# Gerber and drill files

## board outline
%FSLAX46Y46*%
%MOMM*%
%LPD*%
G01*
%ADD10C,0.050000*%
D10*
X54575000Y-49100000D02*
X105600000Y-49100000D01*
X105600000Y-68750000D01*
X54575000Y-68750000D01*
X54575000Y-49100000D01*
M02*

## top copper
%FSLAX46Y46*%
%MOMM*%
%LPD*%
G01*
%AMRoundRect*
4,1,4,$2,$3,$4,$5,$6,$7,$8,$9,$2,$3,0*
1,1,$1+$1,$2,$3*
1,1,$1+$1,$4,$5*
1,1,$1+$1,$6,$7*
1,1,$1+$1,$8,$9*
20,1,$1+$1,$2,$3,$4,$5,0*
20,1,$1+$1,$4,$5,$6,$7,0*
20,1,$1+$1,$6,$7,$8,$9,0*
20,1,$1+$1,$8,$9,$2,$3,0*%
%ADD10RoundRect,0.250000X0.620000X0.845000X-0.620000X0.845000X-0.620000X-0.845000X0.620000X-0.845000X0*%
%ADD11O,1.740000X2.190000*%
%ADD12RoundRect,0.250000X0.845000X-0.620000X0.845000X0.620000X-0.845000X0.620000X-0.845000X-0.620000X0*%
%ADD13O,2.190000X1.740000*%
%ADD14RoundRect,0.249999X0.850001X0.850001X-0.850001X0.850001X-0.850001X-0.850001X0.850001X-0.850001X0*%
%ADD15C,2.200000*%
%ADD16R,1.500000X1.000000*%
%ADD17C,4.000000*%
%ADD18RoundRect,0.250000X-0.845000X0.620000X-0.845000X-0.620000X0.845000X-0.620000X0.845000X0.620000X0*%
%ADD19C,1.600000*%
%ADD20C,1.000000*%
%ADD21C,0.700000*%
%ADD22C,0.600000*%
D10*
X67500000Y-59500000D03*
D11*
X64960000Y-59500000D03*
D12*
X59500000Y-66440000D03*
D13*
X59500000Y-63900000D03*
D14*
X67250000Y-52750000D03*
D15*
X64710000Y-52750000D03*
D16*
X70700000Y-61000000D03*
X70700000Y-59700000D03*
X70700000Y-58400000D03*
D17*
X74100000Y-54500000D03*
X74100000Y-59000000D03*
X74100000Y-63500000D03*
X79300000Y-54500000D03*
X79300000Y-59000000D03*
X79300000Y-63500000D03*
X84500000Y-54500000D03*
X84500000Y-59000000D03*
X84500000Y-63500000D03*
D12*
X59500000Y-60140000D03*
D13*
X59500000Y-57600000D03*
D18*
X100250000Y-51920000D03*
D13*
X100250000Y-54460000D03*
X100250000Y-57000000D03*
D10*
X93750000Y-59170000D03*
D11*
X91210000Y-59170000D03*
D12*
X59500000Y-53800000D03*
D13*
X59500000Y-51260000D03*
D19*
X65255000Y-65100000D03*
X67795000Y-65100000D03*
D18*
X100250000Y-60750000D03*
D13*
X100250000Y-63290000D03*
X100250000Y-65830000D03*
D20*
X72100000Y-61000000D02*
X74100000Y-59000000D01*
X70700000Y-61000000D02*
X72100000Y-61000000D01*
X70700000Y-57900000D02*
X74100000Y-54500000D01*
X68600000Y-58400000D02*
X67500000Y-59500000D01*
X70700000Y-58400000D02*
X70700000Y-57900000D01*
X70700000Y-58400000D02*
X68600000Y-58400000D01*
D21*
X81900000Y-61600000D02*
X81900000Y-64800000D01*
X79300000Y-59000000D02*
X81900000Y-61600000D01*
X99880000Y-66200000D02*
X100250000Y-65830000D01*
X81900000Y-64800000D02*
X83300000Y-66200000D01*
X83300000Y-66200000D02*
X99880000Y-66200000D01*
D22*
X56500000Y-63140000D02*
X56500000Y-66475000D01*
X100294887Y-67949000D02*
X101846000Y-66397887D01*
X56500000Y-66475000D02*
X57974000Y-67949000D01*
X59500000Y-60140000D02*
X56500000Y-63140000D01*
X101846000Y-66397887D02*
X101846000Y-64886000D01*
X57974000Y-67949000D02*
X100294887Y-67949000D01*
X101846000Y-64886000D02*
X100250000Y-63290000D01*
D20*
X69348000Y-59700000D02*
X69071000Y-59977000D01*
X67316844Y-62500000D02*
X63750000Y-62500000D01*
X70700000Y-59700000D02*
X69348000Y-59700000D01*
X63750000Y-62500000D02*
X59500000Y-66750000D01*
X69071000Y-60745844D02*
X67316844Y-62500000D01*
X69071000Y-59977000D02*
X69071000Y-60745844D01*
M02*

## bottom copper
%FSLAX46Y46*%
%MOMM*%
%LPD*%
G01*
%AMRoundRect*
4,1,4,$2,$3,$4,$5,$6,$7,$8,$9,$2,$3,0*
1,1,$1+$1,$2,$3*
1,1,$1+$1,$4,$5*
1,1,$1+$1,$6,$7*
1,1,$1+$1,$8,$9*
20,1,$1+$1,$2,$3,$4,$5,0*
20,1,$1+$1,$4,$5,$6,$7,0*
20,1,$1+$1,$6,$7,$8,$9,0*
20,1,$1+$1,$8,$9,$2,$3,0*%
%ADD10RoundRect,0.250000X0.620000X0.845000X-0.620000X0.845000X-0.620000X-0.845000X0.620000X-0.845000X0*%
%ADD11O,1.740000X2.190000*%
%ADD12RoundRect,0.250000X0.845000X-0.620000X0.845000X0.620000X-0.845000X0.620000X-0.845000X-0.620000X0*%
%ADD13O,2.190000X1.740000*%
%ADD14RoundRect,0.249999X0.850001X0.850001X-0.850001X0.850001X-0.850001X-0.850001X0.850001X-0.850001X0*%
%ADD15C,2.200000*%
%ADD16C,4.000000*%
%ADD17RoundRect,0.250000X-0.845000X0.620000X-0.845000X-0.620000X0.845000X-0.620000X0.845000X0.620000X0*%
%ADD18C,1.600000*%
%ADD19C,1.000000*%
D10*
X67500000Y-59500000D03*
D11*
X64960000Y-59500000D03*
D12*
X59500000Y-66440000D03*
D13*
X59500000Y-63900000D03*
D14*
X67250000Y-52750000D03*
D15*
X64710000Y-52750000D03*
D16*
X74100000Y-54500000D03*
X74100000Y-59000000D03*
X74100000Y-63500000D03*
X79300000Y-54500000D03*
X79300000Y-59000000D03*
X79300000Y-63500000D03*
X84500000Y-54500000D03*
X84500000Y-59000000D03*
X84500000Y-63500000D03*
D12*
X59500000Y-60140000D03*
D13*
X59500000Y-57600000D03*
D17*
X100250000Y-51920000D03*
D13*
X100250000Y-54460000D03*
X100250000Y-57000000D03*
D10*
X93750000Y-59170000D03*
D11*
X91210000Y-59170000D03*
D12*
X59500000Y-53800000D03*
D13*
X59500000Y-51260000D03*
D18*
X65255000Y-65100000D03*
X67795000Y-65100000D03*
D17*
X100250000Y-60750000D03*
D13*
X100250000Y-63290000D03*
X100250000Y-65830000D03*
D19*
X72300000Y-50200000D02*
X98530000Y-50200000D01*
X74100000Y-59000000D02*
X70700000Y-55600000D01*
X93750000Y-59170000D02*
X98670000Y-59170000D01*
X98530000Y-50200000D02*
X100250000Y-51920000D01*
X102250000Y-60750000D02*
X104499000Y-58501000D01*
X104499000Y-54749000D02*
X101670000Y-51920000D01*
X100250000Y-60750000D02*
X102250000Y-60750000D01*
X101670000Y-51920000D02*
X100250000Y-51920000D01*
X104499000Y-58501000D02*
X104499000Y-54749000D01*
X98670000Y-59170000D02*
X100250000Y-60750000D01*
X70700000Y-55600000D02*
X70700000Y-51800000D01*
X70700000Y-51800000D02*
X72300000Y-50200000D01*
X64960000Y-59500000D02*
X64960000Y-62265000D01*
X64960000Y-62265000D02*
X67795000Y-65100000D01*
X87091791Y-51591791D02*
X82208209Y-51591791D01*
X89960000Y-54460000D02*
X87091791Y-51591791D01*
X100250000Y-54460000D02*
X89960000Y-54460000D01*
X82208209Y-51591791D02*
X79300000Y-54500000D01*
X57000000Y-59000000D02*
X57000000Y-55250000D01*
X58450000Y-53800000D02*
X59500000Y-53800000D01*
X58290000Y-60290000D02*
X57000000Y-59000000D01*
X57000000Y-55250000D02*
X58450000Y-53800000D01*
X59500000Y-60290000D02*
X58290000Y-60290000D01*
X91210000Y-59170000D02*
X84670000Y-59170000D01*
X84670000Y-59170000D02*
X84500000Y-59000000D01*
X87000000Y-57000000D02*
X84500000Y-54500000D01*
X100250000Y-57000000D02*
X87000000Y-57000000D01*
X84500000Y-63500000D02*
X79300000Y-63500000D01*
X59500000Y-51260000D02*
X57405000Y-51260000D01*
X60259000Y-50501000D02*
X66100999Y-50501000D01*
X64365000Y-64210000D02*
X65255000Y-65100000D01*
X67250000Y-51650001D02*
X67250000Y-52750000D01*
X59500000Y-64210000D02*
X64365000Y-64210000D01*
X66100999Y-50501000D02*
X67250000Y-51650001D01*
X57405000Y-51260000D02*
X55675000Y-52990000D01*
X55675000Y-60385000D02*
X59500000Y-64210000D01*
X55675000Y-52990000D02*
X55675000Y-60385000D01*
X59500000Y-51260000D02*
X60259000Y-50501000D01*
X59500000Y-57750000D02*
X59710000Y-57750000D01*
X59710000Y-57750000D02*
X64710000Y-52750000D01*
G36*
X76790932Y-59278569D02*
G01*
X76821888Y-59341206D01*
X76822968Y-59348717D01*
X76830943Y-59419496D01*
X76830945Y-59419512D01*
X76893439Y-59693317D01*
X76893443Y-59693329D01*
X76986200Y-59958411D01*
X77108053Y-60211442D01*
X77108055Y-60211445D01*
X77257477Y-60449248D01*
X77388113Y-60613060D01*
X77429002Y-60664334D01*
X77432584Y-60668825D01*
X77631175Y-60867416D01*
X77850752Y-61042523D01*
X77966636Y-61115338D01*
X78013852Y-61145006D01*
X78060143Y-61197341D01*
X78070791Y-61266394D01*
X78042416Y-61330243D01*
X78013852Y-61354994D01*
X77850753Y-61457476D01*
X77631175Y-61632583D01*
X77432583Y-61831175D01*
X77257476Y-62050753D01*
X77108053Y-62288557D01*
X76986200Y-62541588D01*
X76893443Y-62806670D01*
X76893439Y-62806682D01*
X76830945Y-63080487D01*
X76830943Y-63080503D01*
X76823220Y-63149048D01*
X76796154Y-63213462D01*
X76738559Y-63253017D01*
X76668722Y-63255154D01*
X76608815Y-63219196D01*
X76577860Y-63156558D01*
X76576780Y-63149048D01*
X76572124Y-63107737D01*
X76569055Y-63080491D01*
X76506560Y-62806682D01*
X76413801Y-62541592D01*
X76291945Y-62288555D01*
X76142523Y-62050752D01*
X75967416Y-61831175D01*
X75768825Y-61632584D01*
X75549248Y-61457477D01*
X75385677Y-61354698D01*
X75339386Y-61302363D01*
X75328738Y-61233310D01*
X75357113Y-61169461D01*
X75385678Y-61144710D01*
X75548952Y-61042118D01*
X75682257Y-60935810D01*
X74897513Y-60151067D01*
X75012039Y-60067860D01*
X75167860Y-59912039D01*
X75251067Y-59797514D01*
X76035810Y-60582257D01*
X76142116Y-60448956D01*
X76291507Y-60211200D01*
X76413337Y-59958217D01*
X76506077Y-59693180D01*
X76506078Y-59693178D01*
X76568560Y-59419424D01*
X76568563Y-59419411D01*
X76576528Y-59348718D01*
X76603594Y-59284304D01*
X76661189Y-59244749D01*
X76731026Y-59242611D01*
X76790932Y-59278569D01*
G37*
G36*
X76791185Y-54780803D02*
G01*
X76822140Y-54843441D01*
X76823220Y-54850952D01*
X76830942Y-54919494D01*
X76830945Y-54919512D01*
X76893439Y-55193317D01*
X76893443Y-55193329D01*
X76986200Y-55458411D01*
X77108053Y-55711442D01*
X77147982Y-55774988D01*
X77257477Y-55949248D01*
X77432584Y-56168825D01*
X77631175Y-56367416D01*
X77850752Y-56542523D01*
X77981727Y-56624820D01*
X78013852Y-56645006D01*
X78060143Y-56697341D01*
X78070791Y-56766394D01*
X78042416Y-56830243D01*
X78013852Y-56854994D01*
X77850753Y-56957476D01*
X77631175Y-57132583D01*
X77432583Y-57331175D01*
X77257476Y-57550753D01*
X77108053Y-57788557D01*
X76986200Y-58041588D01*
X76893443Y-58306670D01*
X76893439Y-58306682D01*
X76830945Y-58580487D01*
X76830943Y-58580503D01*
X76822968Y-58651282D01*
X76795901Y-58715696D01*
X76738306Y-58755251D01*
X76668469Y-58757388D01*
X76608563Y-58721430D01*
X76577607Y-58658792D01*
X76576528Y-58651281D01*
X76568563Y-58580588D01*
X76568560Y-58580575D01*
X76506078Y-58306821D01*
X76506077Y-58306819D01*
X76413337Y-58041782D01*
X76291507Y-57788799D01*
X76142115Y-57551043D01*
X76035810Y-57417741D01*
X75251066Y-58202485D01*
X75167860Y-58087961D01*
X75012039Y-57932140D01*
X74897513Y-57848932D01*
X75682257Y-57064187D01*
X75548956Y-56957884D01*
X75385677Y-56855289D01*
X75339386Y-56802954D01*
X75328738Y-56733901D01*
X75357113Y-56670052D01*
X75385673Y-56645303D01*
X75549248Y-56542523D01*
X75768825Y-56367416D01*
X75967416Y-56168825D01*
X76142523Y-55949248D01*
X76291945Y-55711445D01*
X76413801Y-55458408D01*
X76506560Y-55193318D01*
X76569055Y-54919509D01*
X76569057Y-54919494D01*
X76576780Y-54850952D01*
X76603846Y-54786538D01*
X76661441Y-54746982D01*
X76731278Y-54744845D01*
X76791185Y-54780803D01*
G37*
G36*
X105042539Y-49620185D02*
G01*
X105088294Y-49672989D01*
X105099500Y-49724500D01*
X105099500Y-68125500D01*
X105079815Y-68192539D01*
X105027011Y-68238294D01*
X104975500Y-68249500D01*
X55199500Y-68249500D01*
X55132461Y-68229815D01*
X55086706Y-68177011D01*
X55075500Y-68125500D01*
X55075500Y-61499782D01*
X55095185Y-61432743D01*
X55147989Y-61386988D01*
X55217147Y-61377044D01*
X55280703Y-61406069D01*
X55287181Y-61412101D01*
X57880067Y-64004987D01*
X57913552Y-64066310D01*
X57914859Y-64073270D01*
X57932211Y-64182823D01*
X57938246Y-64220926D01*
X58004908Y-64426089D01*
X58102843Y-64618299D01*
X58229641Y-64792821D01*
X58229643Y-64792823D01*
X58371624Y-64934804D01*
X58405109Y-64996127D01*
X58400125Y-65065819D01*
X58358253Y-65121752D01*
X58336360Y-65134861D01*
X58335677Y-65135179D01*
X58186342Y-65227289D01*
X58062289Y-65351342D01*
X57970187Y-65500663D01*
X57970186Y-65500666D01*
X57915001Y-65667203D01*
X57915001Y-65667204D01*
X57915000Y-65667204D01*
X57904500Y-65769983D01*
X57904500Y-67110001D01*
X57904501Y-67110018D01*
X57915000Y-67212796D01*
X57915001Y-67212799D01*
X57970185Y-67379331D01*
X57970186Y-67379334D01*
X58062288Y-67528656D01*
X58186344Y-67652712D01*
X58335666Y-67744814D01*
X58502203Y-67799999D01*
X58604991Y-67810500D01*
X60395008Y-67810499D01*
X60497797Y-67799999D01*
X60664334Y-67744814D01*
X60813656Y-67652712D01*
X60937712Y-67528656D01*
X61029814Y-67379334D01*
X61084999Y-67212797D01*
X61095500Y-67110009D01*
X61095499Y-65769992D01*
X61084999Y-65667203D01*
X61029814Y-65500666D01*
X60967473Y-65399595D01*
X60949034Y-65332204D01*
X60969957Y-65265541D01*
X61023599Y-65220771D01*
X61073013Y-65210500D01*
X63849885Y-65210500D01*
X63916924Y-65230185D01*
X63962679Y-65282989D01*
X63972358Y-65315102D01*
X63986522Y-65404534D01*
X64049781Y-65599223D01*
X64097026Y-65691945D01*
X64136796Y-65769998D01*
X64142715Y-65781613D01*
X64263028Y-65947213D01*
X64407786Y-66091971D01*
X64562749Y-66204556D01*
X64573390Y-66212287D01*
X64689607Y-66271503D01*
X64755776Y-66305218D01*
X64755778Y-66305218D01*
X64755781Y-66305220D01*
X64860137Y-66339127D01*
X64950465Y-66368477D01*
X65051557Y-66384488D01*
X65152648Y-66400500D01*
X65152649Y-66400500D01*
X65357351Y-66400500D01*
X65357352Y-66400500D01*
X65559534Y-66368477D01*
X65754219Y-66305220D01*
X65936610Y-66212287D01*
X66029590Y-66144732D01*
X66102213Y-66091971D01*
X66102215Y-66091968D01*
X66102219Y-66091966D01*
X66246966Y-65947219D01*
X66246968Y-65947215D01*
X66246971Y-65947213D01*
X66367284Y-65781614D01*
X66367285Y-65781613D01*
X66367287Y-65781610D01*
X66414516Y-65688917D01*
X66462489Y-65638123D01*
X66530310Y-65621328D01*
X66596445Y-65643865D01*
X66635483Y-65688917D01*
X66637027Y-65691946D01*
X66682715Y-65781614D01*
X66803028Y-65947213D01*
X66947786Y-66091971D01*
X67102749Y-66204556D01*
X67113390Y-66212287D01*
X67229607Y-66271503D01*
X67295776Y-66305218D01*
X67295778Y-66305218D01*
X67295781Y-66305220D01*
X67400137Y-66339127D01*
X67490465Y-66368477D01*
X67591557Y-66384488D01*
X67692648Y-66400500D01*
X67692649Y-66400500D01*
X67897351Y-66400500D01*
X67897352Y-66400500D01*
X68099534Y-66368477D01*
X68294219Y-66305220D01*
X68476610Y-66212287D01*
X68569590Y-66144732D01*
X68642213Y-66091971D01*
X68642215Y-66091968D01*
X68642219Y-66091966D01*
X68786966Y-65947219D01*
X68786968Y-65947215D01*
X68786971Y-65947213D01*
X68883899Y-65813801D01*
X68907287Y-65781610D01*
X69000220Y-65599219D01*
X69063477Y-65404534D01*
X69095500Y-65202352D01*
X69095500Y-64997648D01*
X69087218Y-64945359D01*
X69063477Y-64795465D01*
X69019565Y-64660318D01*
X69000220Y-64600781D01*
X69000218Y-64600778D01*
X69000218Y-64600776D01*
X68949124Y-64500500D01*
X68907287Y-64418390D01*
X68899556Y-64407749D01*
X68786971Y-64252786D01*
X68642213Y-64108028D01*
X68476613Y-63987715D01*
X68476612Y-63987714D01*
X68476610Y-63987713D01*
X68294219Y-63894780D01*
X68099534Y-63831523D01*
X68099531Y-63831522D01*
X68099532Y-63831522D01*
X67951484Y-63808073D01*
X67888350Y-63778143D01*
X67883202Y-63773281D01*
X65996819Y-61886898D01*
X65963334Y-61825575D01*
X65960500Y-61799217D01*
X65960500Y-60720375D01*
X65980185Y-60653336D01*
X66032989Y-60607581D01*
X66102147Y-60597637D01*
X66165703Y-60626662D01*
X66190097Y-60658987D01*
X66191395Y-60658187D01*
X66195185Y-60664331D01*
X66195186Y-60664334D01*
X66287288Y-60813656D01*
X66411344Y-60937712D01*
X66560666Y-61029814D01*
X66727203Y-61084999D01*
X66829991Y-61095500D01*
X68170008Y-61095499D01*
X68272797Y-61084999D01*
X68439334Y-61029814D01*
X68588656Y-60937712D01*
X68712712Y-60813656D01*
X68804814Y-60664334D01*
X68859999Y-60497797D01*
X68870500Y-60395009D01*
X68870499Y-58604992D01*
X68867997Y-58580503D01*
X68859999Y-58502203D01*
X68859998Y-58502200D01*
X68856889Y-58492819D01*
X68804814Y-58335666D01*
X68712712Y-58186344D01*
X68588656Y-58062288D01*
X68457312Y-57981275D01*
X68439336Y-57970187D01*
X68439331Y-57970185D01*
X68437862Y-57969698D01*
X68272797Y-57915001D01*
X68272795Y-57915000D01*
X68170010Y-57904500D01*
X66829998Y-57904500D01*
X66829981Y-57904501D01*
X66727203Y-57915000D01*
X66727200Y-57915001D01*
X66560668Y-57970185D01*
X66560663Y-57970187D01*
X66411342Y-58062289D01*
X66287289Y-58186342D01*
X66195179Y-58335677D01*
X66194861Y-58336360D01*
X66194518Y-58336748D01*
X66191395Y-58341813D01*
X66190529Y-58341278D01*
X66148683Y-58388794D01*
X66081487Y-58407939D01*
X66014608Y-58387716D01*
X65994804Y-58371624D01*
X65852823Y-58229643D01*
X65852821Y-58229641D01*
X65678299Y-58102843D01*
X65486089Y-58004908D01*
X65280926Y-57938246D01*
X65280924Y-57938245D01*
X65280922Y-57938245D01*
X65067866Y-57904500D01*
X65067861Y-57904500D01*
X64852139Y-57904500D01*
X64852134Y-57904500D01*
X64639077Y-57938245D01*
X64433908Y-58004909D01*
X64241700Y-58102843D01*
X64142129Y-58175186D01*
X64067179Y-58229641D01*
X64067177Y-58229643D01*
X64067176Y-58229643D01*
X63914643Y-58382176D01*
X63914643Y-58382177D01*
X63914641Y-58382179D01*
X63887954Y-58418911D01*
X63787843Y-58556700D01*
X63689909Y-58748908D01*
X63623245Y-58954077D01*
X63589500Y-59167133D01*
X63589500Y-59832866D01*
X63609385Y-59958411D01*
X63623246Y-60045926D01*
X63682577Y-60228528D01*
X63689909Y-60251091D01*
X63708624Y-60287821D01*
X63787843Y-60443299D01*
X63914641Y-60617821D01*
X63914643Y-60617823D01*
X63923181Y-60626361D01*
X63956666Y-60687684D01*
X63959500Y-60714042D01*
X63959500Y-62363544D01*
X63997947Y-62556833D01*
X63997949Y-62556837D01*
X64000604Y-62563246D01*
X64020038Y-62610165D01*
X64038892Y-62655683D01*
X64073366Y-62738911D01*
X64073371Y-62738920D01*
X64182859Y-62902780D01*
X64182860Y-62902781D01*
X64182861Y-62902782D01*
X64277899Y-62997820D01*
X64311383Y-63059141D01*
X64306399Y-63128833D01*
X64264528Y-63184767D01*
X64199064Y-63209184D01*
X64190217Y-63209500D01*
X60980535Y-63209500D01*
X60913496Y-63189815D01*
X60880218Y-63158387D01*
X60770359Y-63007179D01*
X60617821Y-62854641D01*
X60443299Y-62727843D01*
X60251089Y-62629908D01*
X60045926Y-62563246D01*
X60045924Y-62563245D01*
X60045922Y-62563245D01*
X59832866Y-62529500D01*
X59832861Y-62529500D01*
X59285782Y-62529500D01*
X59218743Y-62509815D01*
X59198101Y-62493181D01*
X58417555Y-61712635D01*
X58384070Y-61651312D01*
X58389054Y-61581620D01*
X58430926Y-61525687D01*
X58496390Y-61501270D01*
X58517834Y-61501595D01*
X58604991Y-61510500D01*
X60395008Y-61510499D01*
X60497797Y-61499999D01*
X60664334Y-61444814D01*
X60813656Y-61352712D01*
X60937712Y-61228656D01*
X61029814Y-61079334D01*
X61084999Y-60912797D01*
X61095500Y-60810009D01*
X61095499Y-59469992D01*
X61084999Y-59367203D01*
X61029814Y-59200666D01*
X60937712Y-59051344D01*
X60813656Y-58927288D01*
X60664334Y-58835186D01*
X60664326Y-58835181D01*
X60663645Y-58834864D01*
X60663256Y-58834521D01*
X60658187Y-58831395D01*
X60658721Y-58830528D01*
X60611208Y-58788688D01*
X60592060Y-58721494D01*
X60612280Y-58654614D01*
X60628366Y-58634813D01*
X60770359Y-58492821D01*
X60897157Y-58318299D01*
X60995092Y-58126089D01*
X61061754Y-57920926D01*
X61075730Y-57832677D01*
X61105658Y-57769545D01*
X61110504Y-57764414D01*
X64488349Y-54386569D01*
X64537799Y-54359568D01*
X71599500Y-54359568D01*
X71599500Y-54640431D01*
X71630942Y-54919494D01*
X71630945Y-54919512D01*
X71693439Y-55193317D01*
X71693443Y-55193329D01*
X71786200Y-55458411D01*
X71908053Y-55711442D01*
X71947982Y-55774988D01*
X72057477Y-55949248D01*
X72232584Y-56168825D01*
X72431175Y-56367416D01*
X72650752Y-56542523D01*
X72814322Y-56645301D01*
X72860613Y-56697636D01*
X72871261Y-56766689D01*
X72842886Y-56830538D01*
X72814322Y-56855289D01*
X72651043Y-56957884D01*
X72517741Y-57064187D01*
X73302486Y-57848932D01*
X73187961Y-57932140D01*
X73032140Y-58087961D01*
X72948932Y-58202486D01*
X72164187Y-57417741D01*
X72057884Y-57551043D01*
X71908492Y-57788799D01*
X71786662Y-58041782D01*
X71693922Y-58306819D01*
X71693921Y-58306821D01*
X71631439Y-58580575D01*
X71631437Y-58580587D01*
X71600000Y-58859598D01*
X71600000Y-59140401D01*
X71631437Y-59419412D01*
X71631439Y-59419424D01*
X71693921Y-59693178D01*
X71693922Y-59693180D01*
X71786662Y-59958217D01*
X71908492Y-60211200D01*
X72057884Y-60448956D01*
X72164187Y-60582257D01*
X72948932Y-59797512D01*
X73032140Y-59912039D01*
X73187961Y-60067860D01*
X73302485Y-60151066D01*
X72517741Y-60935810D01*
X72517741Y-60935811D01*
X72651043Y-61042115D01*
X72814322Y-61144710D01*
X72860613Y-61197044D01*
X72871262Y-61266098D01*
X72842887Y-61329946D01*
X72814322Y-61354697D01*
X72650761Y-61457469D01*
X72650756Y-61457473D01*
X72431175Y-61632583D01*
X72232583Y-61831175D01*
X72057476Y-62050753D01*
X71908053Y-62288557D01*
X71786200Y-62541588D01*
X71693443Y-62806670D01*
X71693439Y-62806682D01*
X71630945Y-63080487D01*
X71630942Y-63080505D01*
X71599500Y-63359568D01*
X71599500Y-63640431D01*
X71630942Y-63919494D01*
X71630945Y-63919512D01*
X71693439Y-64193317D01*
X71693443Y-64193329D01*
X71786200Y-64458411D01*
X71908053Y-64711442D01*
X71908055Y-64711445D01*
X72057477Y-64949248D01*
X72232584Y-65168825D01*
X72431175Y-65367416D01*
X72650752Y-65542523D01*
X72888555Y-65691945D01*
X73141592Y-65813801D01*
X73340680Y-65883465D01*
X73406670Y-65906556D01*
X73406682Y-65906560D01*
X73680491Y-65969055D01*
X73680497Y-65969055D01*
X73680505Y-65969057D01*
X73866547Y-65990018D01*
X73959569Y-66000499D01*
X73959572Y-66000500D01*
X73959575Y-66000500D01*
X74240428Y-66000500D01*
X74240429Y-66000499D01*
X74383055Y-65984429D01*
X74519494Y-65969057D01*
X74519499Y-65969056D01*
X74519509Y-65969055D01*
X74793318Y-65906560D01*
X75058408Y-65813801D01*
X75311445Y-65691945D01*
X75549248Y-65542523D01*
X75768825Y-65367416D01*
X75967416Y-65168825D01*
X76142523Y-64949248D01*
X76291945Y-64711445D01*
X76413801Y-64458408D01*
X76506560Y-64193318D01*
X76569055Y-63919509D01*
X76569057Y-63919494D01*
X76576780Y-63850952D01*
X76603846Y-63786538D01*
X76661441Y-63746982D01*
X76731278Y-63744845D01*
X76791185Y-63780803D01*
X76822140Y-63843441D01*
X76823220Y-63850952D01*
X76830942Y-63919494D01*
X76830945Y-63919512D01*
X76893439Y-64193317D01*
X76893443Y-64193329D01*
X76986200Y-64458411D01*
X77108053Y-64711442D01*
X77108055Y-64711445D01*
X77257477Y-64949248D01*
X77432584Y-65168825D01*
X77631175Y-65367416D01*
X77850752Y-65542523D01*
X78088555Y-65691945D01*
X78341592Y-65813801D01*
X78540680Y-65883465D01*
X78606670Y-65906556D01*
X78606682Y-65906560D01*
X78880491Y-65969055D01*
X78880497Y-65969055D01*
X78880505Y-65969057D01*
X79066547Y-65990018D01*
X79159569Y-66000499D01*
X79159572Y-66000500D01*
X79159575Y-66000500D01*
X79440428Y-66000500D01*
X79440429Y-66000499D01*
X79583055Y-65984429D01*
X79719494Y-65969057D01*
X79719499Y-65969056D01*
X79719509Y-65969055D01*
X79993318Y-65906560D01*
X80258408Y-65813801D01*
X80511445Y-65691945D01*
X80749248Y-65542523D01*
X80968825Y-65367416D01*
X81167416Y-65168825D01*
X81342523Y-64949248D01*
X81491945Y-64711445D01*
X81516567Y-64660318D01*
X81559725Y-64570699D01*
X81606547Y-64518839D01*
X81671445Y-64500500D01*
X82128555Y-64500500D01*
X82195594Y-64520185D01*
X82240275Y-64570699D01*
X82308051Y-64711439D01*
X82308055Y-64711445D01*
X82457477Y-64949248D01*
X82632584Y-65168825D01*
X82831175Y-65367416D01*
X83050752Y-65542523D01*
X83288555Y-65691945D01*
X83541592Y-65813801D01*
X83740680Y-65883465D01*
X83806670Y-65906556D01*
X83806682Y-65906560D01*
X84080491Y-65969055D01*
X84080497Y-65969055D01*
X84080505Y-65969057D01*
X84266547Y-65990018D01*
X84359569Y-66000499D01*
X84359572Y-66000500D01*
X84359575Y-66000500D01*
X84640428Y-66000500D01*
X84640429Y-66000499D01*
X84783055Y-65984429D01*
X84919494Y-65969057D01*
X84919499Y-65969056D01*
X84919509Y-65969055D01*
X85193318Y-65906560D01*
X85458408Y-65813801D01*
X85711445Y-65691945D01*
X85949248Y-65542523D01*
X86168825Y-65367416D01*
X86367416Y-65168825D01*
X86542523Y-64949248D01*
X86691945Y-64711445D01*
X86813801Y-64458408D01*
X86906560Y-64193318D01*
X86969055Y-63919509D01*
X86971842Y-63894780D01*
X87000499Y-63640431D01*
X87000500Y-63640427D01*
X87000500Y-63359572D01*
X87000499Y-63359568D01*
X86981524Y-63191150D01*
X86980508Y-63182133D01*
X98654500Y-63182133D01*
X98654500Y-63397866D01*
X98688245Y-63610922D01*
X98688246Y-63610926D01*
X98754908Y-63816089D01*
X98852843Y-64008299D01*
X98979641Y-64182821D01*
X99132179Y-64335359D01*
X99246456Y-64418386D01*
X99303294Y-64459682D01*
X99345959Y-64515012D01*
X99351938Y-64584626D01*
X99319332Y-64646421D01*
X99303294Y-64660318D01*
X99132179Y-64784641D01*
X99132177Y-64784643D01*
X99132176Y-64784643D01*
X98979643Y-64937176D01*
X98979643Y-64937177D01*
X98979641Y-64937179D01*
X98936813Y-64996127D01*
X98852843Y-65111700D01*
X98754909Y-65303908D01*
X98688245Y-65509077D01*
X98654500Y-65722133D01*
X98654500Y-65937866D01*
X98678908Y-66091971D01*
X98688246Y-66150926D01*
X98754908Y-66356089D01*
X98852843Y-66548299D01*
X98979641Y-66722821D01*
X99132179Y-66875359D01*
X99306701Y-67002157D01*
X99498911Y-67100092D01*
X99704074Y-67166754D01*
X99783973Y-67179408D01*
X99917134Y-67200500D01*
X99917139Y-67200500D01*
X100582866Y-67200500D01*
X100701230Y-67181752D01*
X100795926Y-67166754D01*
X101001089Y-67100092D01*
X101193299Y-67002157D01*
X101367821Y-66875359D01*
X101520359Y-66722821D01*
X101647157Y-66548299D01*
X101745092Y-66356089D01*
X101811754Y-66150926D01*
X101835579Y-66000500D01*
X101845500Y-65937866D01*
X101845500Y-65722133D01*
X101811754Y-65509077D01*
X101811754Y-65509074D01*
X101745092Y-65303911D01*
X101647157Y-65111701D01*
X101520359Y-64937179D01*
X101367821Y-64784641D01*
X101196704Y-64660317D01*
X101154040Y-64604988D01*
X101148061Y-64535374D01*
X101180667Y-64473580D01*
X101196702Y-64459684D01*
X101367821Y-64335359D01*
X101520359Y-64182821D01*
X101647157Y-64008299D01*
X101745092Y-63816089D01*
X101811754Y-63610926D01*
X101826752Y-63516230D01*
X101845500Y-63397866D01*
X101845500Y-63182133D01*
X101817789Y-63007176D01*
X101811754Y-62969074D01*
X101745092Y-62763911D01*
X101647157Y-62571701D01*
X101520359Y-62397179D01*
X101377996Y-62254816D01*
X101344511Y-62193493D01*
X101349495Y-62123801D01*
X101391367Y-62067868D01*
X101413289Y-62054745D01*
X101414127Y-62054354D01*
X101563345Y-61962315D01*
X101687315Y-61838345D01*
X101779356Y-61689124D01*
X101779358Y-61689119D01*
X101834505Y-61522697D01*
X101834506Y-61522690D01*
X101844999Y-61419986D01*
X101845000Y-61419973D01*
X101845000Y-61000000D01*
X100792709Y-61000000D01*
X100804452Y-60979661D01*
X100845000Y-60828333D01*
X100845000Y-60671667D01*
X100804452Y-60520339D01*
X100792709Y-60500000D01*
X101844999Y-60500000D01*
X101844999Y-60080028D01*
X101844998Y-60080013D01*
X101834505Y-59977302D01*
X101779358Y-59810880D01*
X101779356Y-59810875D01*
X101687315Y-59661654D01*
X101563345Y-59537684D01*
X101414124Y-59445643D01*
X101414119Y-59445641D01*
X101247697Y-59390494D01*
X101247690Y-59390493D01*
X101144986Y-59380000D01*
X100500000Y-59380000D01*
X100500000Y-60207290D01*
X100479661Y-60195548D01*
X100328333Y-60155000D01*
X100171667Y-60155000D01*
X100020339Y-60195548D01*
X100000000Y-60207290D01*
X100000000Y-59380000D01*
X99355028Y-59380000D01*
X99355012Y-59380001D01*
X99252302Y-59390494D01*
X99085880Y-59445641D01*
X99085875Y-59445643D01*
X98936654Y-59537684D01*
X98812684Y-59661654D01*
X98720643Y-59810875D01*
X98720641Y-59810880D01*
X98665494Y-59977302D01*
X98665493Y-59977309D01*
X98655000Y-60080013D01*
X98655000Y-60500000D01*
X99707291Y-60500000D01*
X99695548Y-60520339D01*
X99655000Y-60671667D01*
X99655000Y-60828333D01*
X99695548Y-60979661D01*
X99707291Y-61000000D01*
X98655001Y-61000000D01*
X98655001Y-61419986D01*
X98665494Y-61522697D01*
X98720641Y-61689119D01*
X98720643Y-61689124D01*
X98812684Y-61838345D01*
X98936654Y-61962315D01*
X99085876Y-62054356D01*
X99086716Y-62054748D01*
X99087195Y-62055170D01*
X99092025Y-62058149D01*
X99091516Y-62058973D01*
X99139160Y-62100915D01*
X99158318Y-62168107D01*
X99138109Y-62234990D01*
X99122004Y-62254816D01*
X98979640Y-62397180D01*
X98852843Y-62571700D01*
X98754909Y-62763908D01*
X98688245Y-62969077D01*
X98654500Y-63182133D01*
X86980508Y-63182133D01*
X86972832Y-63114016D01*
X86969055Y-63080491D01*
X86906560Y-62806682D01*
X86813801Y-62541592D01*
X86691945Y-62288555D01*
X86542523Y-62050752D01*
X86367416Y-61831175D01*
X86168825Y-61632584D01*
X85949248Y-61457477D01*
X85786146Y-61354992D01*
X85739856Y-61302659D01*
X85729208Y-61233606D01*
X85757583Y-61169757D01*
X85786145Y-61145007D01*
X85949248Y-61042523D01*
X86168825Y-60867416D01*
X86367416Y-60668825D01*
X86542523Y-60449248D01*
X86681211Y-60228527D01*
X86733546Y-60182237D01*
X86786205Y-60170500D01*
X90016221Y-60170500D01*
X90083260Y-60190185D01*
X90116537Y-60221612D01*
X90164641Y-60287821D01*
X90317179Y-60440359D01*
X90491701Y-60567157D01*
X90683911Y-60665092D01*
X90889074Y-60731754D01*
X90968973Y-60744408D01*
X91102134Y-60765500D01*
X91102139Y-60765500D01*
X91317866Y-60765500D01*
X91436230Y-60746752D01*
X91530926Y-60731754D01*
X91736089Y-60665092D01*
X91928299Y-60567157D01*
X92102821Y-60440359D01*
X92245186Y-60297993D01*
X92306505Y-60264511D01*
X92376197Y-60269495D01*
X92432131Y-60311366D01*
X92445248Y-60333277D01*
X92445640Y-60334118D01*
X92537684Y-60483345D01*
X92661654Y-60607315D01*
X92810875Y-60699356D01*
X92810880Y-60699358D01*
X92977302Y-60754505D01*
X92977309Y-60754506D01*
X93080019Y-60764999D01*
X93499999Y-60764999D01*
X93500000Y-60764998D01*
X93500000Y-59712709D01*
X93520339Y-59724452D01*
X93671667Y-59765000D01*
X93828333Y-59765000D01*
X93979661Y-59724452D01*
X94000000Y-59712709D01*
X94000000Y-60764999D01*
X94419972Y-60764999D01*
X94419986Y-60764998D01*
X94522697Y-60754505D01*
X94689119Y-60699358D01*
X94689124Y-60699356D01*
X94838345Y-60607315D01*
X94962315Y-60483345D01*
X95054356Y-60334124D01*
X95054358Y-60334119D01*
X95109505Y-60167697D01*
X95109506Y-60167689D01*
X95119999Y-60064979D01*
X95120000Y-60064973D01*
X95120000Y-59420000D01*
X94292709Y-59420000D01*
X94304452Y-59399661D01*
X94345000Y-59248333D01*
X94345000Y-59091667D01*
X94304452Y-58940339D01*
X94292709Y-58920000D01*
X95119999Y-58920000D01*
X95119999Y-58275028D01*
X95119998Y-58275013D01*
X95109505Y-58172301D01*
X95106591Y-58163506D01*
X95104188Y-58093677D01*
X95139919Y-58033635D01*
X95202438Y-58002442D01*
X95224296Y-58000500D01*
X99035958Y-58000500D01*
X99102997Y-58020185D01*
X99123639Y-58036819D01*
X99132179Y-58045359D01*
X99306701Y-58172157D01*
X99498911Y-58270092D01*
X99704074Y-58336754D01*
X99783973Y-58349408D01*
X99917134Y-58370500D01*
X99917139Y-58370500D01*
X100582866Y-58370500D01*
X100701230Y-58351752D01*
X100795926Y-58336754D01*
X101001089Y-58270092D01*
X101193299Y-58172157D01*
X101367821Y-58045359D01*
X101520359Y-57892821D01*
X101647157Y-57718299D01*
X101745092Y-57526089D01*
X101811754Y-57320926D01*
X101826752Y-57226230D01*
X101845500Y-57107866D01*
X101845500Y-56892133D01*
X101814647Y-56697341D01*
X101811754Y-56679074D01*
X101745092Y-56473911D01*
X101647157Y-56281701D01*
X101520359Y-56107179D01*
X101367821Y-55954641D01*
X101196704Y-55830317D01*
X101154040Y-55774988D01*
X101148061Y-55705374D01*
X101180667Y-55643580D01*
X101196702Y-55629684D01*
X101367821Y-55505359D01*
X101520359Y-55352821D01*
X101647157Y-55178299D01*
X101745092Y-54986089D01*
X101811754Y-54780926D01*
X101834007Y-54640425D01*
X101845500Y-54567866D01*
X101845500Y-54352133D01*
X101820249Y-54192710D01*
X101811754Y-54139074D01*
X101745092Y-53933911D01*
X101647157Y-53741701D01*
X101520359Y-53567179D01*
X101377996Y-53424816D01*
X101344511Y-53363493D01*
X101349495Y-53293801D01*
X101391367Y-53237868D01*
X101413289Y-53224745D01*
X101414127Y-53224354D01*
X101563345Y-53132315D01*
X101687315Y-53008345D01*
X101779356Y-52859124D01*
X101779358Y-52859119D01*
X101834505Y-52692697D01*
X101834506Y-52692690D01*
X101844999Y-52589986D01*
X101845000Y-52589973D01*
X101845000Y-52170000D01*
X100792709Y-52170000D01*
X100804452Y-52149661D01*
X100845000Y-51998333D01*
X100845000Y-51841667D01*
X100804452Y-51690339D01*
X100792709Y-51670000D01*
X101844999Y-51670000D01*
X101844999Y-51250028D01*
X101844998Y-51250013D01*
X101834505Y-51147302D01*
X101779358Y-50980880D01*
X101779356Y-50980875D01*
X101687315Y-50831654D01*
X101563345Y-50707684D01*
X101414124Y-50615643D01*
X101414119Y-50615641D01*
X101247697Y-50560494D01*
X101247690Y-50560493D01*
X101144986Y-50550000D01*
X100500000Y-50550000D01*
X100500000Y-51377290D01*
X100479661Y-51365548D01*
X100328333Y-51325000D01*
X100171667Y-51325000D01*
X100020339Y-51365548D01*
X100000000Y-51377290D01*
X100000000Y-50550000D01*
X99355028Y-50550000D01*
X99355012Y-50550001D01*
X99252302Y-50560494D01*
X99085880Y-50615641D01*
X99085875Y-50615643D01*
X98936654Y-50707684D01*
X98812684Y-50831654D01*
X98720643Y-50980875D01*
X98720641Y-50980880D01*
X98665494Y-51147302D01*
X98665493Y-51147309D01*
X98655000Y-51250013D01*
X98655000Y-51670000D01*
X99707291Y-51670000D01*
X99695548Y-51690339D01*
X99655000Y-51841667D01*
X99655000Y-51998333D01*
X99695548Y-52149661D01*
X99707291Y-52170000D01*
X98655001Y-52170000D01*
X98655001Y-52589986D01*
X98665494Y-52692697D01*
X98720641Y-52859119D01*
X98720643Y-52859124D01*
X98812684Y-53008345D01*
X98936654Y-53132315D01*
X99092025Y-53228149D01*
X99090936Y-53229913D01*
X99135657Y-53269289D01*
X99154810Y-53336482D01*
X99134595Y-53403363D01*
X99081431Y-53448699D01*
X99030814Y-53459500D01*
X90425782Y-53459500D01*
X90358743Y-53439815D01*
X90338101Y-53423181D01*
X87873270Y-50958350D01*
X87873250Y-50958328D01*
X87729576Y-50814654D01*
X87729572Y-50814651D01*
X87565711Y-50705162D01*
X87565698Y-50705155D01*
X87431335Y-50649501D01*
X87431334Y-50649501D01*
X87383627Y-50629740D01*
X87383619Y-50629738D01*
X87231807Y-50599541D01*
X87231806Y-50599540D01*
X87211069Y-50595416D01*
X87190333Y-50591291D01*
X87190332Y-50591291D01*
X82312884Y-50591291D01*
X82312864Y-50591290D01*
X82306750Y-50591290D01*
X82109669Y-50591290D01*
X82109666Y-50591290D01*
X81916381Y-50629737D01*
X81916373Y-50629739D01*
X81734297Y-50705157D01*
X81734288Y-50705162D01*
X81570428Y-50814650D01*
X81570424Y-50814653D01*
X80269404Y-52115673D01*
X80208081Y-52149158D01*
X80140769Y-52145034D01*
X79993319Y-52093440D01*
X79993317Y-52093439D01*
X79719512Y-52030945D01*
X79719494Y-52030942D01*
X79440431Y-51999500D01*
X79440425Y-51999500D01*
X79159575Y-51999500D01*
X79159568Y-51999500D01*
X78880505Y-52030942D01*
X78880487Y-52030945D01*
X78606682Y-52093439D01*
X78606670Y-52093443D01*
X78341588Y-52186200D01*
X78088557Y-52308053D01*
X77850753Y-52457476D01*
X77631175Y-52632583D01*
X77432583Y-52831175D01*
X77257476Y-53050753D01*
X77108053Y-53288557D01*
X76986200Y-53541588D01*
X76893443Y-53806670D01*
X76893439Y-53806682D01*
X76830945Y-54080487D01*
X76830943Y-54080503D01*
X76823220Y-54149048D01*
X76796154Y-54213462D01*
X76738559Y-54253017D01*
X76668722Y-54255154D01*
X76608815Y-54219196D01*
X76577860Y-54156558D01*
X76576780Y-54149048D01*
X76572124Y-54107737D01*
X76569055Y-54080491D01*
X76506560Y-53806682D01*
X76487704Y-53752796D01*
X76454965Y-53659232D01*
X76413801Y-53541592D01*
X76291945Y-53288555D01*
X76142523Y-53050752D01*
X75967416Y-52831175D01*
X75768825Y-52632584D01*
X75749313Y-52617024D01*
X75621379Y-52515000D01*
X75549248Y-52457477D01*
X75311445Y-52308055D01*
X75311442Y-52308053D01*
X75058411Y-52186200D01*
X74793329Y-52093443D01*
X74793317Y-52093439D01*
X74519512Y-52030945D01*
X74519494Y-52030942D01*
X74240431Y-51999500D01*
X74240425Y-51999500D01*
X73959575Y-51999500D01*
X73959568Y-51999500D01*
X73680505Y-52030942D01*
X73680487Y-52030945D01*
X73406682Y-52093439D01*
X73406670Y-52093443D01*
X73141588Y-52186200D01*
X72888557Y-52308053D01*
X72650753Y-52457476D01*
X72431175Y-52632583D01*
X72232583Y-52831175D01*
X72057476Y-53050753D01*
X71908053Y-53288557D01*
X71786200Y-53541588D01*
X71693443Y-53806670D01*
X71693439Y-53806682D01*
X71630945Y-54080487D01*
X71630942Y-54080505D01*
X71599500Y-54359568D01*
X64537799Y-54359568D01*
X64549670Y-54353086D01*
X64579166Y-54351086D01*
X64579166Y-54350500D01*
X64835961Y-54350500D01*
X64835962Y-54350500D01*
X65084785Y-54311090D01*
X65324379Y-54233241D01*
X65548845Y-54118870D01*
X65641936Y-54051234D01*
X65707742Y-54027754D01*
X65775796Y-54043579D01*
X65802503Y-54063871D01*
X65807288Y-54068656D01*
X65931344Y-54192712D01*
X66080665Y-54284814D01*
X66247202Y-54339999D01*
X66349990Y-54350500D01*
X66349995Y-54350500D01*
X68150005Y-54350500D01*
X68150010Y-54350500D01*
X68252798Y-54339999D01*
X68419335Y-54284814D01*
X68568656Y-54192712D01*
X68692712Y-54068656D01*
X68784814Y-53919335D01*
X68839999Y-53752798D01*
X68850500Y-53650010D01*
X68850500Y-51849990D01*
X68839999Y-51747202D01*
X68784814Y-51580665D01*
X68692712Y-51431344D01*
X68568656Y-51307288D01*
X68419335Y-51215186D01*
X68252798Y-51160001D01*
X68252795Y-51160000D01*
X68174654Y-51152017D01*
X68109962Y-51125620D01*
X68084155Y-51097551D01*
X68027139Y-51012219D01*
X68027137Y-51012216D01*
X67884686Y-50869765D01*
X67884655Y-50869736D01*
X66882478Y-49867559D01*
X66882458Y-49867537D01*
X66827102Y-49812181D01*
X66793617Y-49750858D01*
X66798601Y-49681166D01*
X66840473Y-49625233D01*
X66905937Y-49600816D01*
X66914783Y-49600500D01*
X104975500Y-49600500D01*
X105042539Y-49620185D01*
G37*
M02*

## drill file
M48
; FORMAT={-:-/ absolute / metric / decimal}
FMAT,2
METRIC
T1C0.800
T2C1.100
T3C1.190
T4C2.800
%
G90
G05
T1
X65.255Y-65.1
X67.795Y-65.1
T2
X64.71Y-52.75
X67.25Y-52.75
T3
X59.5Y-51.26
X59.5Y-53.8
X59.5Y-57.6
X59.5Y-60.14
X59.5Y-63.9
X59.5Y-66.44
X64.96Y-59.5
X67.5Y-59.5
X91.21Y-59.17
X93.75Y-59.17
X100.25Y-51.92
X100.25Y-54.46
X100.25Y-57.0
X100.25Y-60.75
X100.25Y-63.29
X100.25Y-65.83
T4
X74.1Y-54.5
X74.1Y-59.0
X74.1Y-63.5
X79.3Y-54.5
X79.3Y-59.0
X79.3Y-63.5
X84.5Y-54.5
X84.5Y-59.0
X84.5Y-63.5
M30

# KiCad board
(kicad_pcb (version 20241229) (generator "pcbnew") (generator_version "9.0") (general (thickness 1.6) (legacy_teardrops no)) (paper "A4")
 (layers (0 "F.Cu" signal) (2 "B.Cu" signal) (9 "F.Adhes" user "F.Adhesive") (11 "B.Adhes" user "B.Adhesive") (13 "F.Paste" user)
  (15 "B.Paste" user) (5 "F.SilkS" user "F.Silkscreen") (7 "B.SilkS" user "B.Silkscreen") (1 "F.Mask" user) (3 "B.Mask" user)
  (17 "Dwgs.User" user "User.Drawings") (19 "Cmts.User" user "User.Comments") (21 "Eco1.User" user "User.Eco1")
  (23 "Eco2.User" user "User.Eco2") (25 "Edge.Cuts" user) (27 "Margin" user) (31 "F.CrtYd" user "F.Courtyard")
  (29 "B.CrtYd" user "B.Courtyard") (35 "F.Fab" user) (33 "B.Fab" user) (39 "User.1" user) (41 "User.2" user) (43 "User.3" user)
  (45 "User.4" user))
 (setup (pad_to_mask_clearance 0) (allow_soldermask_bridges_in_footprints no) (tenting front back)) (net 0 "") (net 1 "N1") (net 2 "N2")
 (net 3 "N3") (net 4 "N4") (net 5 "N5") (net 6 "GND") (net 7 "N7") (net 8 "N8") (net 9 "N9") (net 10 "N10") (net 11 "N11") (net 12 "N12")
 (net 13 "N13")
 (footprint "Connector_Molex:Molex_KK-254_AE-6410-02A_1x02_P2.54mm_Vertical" (layer "F.Cu") (at 67.5 59.5 180)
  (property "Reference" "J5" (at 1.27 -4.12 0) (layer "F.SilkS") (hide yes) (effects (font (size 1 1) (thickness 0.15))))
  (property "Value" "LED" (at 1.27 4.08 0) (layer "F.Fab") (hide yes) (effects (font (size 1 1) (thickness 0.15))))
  (pad "1" thru_hole roundrect (at 0 0 180) (size 1.74 2.19) (drill 1.19) (layers "*.Cu" "*.Mask") (remove_unused_layers no)
   (roundrect_rratio 0.143678) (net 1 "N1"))
  (pad "2" thru_hole oval (at 2.54 0 180) (size 1.74 2.19) (drill 1.19) (layers "*.Cu" "*.Mask") (remove_unused_layers no) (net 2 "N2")))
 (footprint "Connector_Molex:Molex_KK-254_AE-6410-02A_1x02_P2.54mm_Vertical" (layer "F.Cu") (at 59.5 66.44 90)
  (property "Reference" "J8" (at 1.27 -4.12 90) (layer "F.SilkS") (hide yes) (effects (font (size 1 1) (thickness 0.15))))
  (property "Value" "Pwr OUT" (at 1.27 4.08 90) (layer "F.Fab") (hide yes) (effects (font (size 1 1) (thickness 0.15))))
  (pad "1" thru_hole roundrect (at 0 0 90) (size 1.74 2.19) (drill 1.19) (layers "*.Cu" "*.Mask") (remove_unused_layers no)
   (roundrect_rratio 0.143678) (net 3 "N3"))
  (pad "2" thru_hole oval (at 2.54 0 90) (size 1.74 2.19) (drill 1.19) (layers "*.Cu" "*.Mask") (remove_unused_layers no) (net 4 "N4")))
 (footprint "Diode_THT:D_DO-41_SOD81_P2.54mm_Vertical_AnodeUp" (layer "F.Cu") (at 67.25 52.75 180)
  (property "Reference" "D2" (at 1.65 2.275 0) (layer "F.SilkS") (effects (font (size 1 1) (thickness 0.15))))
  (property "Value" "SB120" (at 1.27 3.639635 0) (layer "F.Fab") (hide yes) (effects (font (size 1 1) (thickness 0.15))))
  (pad "1" thru_hole roundrect (at 0 0 180) (size 2.2 2.2) (drill 1.1) (layers "*.Cu" "*.Mask") (remove_unused_layers no)
   (roundrect_rratio 0.113636) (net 4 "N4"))
  (pad "2" thru_hole circle (at 2.54 0 180) (size 2.2 2.2) (drill 1.1) (layers "*.Cu" "*.Mask") (remove_unused_layers no) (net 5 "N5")))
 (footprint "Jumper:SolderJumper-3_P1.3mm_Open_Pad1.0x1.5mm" (layer "F.Cu") (at 70.7 59.7 90)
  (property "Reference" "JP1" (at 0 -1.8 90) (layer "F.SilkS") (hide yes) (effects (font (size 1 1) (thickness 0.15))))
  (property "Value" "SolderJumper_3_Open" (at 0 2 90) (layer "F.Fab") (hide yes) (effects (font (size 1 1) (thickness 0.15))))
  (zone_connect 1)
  (pad "1" smd rect (at -1.3 0 90) (size 1 1.5) (layers "F.Cu" "F.Mask") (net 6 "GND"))
  (pad "2" smd rect (at 0 0 90) (size 1 1.5) (layers "F.Cu" "F.Mask") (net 3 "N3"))
  (pad "3" smd rect (at 1.3 0 90) (size 1 1.5) (layers "F.Cu" "F.Mask") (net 1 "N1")))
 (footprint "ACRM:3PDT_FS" (layer "F.Cu") (at 77.1 58)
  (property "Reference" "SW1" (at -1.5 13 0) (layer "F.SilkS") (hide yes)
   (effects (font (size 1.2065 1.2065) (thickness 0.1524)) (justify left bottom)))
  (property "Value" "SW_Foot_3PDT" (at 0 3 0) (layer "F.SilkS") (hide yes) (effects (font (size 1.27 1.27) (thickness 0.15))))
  (pad "A1" thru_hole circle (at -3 -3.5 180) (size 4 4) (drill 2.8) (layers "*.Cu" "*.Mask") (remove_unused_layers no) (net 1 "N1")
   (solder_mask_margin 0.1016))
  (pad "A2" thru_hole circle (at -3 1 180) (size 4 4) (drill 2.8) (layers "*.Cu" "*.Mask") (remove_unused_layers no) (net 6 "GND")
   (solder_mask_margin 0.1016))
  (pad "A3" thru_hole circle (at -3 5.5 180) (size 4 4) (drill 2.8) (layers "*.Cu" "*.Mask") (remove_unused_layers no) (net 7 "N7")
   (solder_mask_margin 0.1016))
  (pad "B1" thru_hole circle (at 2.2 -3.5 180) (size 4 4) (drill 2.8) (layers "*.Cu" "*.Mask") (remove_unused_layers no) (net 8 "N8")
   (solder_mask_margin 0.1016))
  (pad "B2" thru_hole circle (at 2.2 1 180) (size 4 4) (drill 2.8) (layers "*.Cu" "*.Mask") (remove_unused_layers no) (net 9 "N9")
   (solder_mask_margin 0.1016))
  (pad "B3" thru_hole circle (at 2.2 5.5 180) (size 4 4) (drill 2.8) (layers "*.Cu" "*.Mask") (remove_unused_layers no) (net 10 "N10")
   (solder_mask_margin 0.1016))
  (pad "C1" thru_hole circle (at 7.4 -3.5 180) (size 4 4) (drill 2.8) (layers "*.Cu" "*.Mask") (remove_unused_layers no) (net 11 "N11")
   (solder_mask_margin 0.1016))
  (pad "C2" thru_hole circle (at 7.4 1 180) (size 4 4) (drill 2.8) (layers "*.Cu" "*.Mask") (remove_unused_layers no) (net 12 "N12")
   (solder_mask_margin 0.1016))
  (pad "C3" thru_hole circle (at 7.4 5.5 180) (size 4 4) (drill 2.8) (layers "*.Cu" "*.Mask") (remove_unused_layers no) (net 10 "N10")
   (solder_mask_margin 0.1016)))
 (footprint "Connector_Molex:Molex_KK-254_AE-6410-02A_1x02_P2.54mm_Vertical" (layer "F.Cu") (at 59.5 60.14 90)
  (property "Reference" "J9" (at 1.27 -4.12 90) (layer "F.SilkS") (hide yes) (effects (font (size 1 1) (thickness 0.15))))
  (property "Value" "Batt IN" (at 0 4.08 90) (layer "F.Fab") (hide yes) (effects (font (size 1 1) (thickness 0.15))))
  (pad "1" thru_hole roundrect (at 0 0 90) (size 1.74 2.19) (drill 1.19) (layers "*.Cu" "*.Mask") (remove_unused_layers no)
   (roundrect_rratio 0.143678) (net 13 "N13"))
  (pad "2" thru_hole oval (at 2.54 0 90) (size 1.74 2.19) (drill 1.19) (layers "*.Cu" "*.Mask") (remove_unused_layers no) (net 5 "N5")))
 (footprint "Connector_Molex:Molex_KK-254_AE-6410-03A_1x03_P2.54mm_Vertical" (layer "F.Cu") (at 100.25 51.92 -90)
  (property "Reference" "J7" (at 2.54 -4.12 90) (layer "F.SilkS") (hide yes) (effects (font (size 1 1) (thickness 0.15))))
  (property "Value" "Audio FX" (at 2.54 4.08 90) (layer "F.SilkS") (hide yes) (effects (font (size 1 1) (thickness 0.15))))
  (pad "1" thru_hole roundrect (at 0 0 270) (size 1.74 2.19) (drill 1.19) (layers "*.Cu" "*.Mask") (remove_unused_layers no)
   (roundrect_rratio 0.143678) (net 6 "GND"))
  (pad "2" thru_hole oval (at 2.54 0 270) (size 1.74 2.19) (drill 1.19) (layers "*.Cu" "*.Mask") (remove_unused_layers no) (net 8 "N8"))
  (pad "3" thru_hole oval (at 5.08 0 270) (size 1.74 2.19) (drill 1.19) (layers "*.Cu" "*.Mask") (remove_unused_layers no) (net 11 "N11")))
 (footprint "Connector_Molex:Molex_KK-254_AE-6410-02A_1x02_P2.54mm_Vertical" (layer "F.Cu") (at 93.75 59.17 180)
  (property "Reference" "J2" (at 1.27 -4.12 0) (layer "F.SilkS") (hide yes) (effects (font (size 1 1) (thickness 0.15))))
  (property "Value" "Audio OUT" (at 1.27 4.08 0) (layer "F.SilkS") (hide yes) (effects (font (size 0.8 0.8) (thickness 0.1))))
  (pad "1" thru_hole roundrect (at 0 0 180) (size 1.74 2.19) (drill 1.19) (layers "*.Cu" "*.Mask") (remove_unused_layers no)
   (roundrect_rratio 0.143678) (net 6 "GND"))
  (pad "2" thru_hole oval (at 2.54 0 180) (size 1.74 2.19) (drill 1.19) (layers "*.Cu" "*.Mask") (remove_unused_layers no) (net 12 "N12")))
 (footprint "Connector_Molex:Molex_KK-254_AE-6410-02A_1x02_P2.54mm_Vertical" (layer "F.Cu") (at 59.5 53.8 90)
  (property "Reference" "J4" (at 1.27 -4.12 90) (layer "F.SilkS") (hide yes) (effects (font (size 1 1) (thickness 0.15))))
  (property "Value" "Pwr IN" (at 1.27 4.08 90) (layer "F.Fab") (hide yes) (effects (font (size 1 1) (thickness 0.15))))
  (pad "1" thru_hole roundrect (at 0 0 90) (size 1.74 2.19) (drill 1.19) (layers "*.Cu" "*.Mask") (remove_unused_layers no)
   (roundrect_rratio 0.143678) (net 13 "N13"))
  (pad "2" thru_hole oval (at 2.54 0 90) (size 1.74 2.19) (drill 1.19) (layers "*.Cu" "*.Mask") (remove_unused_layers no) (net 4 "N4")))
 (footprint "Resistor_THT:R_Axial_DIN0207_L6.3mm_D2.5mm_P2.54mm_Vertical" (layer "F.Cu") (at 65.255 65.1)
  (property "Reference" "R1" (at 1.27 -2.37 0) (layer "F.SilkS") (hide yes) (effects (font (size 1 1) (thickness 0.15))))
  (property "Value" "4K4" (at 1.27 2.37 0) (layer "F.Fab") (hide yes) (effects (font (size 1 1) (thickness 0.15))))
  (pad "1" thru_hole circle (at 0 0) (size 1.6 1.6) (drill 0.8) (layers "*.Cu" "*.Mask") (remove_unused_layers no) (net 4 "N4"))
  (pad "2" thru_hole circle (at 2.54 0) (size 1.6 1.6) (drill 0.8) (layers "*.Cu" "*.Mask") (remove_unused_layers no) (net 2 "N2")))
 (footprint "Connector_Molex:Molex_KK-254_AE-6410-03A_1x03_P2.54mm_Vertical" (layer "F.Cu") (at 100.25 60.75 -90)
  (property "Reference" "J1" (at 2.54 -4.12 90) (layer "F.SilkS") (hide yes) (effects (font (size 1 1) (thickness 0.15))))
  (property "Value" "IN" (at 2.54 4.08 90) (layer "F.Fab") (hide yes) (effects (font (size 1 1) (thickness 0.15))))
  (pad "1" thru_hole roundrect (at 0 0 270) (size 1.74 2.19) (drill 1.19) (layers "*.Cu" "*.Mask") (remove_unused_layers no)
   (roundrect_rratio 0.143678) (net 6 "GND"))
  (pad "2" thru_hole oval (at 2.54 0 270) (size 1.74 2.19) (drill 1.19) (layers "*.Cu" "*.Mask") (remove_unused_layers no) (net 13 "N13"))
  (pad "3" thru_hole oval (at 5.08 0 270) (size 1.74 2.19) (drill 1.19) (layers "*.Cu" "*.Mask") (remove_unused_layers no) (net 9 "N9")))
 (gr_rect (start 54.575 49.1) (end 105.6 68.75) (stroke (width 0.05) (type default)) (fill no) (layer "Edge.Cuts"))
 (segment (start 72.1 61) (end 74.1 59) (width 1) (layer "F.Cu") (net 6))
 (segment (start 70.7 61) (end 72.1 61) (width 1) (layer "F.Cu") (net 6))
 (segment (start 72.3 50.2) (end 98.53 50.2) (width 1) (layer "B.Cu") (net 6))
 (segment (start 74.1 59) (end 70.7 55.6) (width 1) (layer "B.Cu") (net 6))
 (segment (start 93.75 59.17) (end 98.67 59.17) (width 1) (layer "B.Cu") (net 6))
 (segment (start 98.53 50.2) (end 100.25 51.92) (width 1) (layer "B.Cu") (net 6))
 (segment (start 102.25 60.75) (end 104.499 58.501) (width 1) (layer "B.Cu") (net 6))
 (segment (start 104.499 54.749) (end 101.67 51.92) (width 1) (layer "B.Cu") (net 6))
 (segment (start 100.25 60.75) (end 102.25 60.75) (width 1) (layer "B.Cu") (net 6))
 (segment (start 101.67 51.92) (end 100.25 51.92) (width 1) (layer "B.Cu") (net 6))
 (segment (start 104.499 58.501) (end 104.499 54.749) (width 1) (layer "B.Cu") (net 6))
 (segment (start 98.67 59.17) (end 100.25 60.75) (width 1) (layer "B.Cu") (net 6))
 (segment (start 70.7 55.6) (end 70.7 51.8) (width 1) (layer "B.Cu") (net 6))
 (segment (start 70.7 51.8) (end 72.3 50.2) (width 1) (layer "B.Cu") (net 6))
 (segment (start 64.96 59.5) (end 64.96 62.265) (width 1) (layer "B.Cu") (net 2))
 (segment (start 64.96 62.265) (end 67.795 65.1) (width 1) (layer "B.Cu") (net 2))
 (segment (start 87.091791 51.591791) (end 82.208209 51.591791) (width 1) (layer "B.Cu") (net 8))
 (segment (start 89.96 54.46) (end 87.091791 51.591791) (width 1) (layer "B.Cu") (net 8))
 (segment (start 100.25 54.46) (end 89.96 54.46) (width 1) (layer "B.Cu") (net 8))
 (segment (start 82.208209 51.591791) (end 79.3 54.5) (width 1) (layer "B.Cu") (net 8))
 (segment (start 70.7 57.9) (end 74.1 54.5) (width 1) (layer "F.Cu") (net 1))
 (segment (start 68.6 58.4) (end 67.5 59.5) (width 1) (layer "F.Cu") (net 1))
 (segment (start 70.7 58.4) (end 70.7 57.9) (width 1) (layer "F.Cu") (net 1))
 (segment (start 70.7 58.4) (end 68.6 58.4) (width 1) (layer "F.Cu") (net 1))
 (segment (start 81.9 61.6) (end 81.9 64.8) (width 0.7) (layer "F.Cu") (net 9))
 (segment (start 79.3 59) (end 81.9 61.6) (width 0.7) (layer "F.Cu") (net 9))
 (segment (start 99.88 66.2) (end 100.25 65.83) (width 0.7) (layer "F.Cu") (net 9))
 (segment (start 81.9 64.8) (end 83.3 66.2) (width 0.7) (layer "F.Cu") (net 9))
 (segment (start 83.3 66.2) (end 99.88 66.2) (width 0.7) (layer "F.Cu") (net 9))
 (segment (start 56.5 63.14) (end 56.5 66.475) (width 0.6) (layer "F.Cu") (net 13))
 (segment (start 100.294887 67.949) (end 101.846 66.397887) (width 0.6) (layer "F.Cu") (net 13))
 (segment (start 56.5 66.475) (end 57.974 67.949) (width 0.6) (layer "F.Cu") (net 13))
 (segment (start 59.5 60.14) (end 56.5 63.14) (width 0.6) (layer "F.Cu") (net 13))
 (segment (start 101.846 66.397887) (end 101.846 64.886) (width 0.6) (layer "F.Cu") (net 13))
 (segment (start 57.974 67.949) (end 100.294887 67.949) (width 0.6) (layer "F.Cu") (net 13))
 (segment (start 101.846 64.886) (end 100.25 63.29) (width 0.6) (layer "F.Cu") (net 13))
 (segment (start 57 59) (end 57 55.25) (width 1) (layer "B.Cu") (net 13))
 (segment (start 58.45 53.8) (end 59.5 53.8) (width 1) (layer "B.Cu") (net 13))
 (segment (start 58.29 60.29) (end 57 59) (width 1) (layer "B.Cu") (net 13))
 (segment (start 57 55.25) (end 58.45 53.8) (width 1) (layer "B.Cu") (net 13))
 (segment (start 59.5 60.29) (end 58.29 60.29) (width 1) (layer "B.Cu") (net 13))
 (segment (start 91.21 59.17) (end 84.67 59.17) (width 1) (layer "B.Cu") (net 12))
 (segment (start 84.67 59.17) (end 84.5 59) (width 1) (layer "B.Cu") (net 12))
 (segment (start 87 57) (end 84.5 54.5) (width 1) (layer "B.Cu") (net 11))
 (segment (start 100.25 57) (end 87 57) (width 1) (layer "B.Cu") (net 11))
 (segment (start 84.5 63.5) (end 79.3 63.5) (width 1) (layer "B.Cu") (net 10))
 (segment (start 59.5 51.26) (end 57.405 51.26) (width 1) (layer "B.Cu") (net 4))
 (segment (start 60.259 50.501) (end 66.100999 50.501) (width 1) (layer "B.Cu") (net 4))
 (segment (start 64.365 64.21) (end 65.255 65.1) (width 1) (layer "B.Cu") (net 4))
 (segment (start 67.25 51.650001) (end 67.25 52.75) (width 1) (layer "B.Cu") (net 4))
 (segment (start 59.5 64.21) (end 64.365 64.21) (width 1) (layer "B.Cu") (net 4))
 (segment (start 66.100999 50.501) (end 67.25 51.650001) (width 1) (layer "B.Cu") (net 4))
 (segment (start 57.405 51.26) (end 55.675 52.99) (width 1) (layer "B.Cu") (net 4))
 (segment (start 55.675 60.385) (end 59.5 64.21) (width 1) (layer "B.Cu") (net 4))
 (segment (start 55.675 52.99) (end 55.675 60.385) (width 1) (layer "B.Cu") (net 4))
 (segment (start 59.5 51.26) (end 60.259 50.501) (width 1) (layer "B.Cu") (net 4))
 (segment (start 59.5 57.75) (end 59.71 57.75) (width 1) (layer "B.Cu") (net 5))
 (segment (start 59.71 57.75) (end 64.71 52.75) (width 1) (layer "B.Cu") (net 5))
 (segment (start 69.348 59.7) (end 69.071 59.977) (width 1) (layer "F.Cu") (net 3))
 (segment (start 67.316844 62.5) (end 63.75 62.5) (width 1) (layer "F.Cu") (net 3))
 (segment (start 70.7 59.7) (end 69.348 59.7) (width 1) (layer "F.Cu") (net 3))
 (segment (start 63.75 62.5) (end 59.5 66.75) (width 1) (layer "F.Cu") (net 3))
 (segment (start 69.071 60.745844) (end 67.316844 62.5) (width 1) (layer "F.Cu") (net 3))
 (segment (start 69.071 59.977) (end 69.071 60.745844) (width 1) (layer "F.Cu") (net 3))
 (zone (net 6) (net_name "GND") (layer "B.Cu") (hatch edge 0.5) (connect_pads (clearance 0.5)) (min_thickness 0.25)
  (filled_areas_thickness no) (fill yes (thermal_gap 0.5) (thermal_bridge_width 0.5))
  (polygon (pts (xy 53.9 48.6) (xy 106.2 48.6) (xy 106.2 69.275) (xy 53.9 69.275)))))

